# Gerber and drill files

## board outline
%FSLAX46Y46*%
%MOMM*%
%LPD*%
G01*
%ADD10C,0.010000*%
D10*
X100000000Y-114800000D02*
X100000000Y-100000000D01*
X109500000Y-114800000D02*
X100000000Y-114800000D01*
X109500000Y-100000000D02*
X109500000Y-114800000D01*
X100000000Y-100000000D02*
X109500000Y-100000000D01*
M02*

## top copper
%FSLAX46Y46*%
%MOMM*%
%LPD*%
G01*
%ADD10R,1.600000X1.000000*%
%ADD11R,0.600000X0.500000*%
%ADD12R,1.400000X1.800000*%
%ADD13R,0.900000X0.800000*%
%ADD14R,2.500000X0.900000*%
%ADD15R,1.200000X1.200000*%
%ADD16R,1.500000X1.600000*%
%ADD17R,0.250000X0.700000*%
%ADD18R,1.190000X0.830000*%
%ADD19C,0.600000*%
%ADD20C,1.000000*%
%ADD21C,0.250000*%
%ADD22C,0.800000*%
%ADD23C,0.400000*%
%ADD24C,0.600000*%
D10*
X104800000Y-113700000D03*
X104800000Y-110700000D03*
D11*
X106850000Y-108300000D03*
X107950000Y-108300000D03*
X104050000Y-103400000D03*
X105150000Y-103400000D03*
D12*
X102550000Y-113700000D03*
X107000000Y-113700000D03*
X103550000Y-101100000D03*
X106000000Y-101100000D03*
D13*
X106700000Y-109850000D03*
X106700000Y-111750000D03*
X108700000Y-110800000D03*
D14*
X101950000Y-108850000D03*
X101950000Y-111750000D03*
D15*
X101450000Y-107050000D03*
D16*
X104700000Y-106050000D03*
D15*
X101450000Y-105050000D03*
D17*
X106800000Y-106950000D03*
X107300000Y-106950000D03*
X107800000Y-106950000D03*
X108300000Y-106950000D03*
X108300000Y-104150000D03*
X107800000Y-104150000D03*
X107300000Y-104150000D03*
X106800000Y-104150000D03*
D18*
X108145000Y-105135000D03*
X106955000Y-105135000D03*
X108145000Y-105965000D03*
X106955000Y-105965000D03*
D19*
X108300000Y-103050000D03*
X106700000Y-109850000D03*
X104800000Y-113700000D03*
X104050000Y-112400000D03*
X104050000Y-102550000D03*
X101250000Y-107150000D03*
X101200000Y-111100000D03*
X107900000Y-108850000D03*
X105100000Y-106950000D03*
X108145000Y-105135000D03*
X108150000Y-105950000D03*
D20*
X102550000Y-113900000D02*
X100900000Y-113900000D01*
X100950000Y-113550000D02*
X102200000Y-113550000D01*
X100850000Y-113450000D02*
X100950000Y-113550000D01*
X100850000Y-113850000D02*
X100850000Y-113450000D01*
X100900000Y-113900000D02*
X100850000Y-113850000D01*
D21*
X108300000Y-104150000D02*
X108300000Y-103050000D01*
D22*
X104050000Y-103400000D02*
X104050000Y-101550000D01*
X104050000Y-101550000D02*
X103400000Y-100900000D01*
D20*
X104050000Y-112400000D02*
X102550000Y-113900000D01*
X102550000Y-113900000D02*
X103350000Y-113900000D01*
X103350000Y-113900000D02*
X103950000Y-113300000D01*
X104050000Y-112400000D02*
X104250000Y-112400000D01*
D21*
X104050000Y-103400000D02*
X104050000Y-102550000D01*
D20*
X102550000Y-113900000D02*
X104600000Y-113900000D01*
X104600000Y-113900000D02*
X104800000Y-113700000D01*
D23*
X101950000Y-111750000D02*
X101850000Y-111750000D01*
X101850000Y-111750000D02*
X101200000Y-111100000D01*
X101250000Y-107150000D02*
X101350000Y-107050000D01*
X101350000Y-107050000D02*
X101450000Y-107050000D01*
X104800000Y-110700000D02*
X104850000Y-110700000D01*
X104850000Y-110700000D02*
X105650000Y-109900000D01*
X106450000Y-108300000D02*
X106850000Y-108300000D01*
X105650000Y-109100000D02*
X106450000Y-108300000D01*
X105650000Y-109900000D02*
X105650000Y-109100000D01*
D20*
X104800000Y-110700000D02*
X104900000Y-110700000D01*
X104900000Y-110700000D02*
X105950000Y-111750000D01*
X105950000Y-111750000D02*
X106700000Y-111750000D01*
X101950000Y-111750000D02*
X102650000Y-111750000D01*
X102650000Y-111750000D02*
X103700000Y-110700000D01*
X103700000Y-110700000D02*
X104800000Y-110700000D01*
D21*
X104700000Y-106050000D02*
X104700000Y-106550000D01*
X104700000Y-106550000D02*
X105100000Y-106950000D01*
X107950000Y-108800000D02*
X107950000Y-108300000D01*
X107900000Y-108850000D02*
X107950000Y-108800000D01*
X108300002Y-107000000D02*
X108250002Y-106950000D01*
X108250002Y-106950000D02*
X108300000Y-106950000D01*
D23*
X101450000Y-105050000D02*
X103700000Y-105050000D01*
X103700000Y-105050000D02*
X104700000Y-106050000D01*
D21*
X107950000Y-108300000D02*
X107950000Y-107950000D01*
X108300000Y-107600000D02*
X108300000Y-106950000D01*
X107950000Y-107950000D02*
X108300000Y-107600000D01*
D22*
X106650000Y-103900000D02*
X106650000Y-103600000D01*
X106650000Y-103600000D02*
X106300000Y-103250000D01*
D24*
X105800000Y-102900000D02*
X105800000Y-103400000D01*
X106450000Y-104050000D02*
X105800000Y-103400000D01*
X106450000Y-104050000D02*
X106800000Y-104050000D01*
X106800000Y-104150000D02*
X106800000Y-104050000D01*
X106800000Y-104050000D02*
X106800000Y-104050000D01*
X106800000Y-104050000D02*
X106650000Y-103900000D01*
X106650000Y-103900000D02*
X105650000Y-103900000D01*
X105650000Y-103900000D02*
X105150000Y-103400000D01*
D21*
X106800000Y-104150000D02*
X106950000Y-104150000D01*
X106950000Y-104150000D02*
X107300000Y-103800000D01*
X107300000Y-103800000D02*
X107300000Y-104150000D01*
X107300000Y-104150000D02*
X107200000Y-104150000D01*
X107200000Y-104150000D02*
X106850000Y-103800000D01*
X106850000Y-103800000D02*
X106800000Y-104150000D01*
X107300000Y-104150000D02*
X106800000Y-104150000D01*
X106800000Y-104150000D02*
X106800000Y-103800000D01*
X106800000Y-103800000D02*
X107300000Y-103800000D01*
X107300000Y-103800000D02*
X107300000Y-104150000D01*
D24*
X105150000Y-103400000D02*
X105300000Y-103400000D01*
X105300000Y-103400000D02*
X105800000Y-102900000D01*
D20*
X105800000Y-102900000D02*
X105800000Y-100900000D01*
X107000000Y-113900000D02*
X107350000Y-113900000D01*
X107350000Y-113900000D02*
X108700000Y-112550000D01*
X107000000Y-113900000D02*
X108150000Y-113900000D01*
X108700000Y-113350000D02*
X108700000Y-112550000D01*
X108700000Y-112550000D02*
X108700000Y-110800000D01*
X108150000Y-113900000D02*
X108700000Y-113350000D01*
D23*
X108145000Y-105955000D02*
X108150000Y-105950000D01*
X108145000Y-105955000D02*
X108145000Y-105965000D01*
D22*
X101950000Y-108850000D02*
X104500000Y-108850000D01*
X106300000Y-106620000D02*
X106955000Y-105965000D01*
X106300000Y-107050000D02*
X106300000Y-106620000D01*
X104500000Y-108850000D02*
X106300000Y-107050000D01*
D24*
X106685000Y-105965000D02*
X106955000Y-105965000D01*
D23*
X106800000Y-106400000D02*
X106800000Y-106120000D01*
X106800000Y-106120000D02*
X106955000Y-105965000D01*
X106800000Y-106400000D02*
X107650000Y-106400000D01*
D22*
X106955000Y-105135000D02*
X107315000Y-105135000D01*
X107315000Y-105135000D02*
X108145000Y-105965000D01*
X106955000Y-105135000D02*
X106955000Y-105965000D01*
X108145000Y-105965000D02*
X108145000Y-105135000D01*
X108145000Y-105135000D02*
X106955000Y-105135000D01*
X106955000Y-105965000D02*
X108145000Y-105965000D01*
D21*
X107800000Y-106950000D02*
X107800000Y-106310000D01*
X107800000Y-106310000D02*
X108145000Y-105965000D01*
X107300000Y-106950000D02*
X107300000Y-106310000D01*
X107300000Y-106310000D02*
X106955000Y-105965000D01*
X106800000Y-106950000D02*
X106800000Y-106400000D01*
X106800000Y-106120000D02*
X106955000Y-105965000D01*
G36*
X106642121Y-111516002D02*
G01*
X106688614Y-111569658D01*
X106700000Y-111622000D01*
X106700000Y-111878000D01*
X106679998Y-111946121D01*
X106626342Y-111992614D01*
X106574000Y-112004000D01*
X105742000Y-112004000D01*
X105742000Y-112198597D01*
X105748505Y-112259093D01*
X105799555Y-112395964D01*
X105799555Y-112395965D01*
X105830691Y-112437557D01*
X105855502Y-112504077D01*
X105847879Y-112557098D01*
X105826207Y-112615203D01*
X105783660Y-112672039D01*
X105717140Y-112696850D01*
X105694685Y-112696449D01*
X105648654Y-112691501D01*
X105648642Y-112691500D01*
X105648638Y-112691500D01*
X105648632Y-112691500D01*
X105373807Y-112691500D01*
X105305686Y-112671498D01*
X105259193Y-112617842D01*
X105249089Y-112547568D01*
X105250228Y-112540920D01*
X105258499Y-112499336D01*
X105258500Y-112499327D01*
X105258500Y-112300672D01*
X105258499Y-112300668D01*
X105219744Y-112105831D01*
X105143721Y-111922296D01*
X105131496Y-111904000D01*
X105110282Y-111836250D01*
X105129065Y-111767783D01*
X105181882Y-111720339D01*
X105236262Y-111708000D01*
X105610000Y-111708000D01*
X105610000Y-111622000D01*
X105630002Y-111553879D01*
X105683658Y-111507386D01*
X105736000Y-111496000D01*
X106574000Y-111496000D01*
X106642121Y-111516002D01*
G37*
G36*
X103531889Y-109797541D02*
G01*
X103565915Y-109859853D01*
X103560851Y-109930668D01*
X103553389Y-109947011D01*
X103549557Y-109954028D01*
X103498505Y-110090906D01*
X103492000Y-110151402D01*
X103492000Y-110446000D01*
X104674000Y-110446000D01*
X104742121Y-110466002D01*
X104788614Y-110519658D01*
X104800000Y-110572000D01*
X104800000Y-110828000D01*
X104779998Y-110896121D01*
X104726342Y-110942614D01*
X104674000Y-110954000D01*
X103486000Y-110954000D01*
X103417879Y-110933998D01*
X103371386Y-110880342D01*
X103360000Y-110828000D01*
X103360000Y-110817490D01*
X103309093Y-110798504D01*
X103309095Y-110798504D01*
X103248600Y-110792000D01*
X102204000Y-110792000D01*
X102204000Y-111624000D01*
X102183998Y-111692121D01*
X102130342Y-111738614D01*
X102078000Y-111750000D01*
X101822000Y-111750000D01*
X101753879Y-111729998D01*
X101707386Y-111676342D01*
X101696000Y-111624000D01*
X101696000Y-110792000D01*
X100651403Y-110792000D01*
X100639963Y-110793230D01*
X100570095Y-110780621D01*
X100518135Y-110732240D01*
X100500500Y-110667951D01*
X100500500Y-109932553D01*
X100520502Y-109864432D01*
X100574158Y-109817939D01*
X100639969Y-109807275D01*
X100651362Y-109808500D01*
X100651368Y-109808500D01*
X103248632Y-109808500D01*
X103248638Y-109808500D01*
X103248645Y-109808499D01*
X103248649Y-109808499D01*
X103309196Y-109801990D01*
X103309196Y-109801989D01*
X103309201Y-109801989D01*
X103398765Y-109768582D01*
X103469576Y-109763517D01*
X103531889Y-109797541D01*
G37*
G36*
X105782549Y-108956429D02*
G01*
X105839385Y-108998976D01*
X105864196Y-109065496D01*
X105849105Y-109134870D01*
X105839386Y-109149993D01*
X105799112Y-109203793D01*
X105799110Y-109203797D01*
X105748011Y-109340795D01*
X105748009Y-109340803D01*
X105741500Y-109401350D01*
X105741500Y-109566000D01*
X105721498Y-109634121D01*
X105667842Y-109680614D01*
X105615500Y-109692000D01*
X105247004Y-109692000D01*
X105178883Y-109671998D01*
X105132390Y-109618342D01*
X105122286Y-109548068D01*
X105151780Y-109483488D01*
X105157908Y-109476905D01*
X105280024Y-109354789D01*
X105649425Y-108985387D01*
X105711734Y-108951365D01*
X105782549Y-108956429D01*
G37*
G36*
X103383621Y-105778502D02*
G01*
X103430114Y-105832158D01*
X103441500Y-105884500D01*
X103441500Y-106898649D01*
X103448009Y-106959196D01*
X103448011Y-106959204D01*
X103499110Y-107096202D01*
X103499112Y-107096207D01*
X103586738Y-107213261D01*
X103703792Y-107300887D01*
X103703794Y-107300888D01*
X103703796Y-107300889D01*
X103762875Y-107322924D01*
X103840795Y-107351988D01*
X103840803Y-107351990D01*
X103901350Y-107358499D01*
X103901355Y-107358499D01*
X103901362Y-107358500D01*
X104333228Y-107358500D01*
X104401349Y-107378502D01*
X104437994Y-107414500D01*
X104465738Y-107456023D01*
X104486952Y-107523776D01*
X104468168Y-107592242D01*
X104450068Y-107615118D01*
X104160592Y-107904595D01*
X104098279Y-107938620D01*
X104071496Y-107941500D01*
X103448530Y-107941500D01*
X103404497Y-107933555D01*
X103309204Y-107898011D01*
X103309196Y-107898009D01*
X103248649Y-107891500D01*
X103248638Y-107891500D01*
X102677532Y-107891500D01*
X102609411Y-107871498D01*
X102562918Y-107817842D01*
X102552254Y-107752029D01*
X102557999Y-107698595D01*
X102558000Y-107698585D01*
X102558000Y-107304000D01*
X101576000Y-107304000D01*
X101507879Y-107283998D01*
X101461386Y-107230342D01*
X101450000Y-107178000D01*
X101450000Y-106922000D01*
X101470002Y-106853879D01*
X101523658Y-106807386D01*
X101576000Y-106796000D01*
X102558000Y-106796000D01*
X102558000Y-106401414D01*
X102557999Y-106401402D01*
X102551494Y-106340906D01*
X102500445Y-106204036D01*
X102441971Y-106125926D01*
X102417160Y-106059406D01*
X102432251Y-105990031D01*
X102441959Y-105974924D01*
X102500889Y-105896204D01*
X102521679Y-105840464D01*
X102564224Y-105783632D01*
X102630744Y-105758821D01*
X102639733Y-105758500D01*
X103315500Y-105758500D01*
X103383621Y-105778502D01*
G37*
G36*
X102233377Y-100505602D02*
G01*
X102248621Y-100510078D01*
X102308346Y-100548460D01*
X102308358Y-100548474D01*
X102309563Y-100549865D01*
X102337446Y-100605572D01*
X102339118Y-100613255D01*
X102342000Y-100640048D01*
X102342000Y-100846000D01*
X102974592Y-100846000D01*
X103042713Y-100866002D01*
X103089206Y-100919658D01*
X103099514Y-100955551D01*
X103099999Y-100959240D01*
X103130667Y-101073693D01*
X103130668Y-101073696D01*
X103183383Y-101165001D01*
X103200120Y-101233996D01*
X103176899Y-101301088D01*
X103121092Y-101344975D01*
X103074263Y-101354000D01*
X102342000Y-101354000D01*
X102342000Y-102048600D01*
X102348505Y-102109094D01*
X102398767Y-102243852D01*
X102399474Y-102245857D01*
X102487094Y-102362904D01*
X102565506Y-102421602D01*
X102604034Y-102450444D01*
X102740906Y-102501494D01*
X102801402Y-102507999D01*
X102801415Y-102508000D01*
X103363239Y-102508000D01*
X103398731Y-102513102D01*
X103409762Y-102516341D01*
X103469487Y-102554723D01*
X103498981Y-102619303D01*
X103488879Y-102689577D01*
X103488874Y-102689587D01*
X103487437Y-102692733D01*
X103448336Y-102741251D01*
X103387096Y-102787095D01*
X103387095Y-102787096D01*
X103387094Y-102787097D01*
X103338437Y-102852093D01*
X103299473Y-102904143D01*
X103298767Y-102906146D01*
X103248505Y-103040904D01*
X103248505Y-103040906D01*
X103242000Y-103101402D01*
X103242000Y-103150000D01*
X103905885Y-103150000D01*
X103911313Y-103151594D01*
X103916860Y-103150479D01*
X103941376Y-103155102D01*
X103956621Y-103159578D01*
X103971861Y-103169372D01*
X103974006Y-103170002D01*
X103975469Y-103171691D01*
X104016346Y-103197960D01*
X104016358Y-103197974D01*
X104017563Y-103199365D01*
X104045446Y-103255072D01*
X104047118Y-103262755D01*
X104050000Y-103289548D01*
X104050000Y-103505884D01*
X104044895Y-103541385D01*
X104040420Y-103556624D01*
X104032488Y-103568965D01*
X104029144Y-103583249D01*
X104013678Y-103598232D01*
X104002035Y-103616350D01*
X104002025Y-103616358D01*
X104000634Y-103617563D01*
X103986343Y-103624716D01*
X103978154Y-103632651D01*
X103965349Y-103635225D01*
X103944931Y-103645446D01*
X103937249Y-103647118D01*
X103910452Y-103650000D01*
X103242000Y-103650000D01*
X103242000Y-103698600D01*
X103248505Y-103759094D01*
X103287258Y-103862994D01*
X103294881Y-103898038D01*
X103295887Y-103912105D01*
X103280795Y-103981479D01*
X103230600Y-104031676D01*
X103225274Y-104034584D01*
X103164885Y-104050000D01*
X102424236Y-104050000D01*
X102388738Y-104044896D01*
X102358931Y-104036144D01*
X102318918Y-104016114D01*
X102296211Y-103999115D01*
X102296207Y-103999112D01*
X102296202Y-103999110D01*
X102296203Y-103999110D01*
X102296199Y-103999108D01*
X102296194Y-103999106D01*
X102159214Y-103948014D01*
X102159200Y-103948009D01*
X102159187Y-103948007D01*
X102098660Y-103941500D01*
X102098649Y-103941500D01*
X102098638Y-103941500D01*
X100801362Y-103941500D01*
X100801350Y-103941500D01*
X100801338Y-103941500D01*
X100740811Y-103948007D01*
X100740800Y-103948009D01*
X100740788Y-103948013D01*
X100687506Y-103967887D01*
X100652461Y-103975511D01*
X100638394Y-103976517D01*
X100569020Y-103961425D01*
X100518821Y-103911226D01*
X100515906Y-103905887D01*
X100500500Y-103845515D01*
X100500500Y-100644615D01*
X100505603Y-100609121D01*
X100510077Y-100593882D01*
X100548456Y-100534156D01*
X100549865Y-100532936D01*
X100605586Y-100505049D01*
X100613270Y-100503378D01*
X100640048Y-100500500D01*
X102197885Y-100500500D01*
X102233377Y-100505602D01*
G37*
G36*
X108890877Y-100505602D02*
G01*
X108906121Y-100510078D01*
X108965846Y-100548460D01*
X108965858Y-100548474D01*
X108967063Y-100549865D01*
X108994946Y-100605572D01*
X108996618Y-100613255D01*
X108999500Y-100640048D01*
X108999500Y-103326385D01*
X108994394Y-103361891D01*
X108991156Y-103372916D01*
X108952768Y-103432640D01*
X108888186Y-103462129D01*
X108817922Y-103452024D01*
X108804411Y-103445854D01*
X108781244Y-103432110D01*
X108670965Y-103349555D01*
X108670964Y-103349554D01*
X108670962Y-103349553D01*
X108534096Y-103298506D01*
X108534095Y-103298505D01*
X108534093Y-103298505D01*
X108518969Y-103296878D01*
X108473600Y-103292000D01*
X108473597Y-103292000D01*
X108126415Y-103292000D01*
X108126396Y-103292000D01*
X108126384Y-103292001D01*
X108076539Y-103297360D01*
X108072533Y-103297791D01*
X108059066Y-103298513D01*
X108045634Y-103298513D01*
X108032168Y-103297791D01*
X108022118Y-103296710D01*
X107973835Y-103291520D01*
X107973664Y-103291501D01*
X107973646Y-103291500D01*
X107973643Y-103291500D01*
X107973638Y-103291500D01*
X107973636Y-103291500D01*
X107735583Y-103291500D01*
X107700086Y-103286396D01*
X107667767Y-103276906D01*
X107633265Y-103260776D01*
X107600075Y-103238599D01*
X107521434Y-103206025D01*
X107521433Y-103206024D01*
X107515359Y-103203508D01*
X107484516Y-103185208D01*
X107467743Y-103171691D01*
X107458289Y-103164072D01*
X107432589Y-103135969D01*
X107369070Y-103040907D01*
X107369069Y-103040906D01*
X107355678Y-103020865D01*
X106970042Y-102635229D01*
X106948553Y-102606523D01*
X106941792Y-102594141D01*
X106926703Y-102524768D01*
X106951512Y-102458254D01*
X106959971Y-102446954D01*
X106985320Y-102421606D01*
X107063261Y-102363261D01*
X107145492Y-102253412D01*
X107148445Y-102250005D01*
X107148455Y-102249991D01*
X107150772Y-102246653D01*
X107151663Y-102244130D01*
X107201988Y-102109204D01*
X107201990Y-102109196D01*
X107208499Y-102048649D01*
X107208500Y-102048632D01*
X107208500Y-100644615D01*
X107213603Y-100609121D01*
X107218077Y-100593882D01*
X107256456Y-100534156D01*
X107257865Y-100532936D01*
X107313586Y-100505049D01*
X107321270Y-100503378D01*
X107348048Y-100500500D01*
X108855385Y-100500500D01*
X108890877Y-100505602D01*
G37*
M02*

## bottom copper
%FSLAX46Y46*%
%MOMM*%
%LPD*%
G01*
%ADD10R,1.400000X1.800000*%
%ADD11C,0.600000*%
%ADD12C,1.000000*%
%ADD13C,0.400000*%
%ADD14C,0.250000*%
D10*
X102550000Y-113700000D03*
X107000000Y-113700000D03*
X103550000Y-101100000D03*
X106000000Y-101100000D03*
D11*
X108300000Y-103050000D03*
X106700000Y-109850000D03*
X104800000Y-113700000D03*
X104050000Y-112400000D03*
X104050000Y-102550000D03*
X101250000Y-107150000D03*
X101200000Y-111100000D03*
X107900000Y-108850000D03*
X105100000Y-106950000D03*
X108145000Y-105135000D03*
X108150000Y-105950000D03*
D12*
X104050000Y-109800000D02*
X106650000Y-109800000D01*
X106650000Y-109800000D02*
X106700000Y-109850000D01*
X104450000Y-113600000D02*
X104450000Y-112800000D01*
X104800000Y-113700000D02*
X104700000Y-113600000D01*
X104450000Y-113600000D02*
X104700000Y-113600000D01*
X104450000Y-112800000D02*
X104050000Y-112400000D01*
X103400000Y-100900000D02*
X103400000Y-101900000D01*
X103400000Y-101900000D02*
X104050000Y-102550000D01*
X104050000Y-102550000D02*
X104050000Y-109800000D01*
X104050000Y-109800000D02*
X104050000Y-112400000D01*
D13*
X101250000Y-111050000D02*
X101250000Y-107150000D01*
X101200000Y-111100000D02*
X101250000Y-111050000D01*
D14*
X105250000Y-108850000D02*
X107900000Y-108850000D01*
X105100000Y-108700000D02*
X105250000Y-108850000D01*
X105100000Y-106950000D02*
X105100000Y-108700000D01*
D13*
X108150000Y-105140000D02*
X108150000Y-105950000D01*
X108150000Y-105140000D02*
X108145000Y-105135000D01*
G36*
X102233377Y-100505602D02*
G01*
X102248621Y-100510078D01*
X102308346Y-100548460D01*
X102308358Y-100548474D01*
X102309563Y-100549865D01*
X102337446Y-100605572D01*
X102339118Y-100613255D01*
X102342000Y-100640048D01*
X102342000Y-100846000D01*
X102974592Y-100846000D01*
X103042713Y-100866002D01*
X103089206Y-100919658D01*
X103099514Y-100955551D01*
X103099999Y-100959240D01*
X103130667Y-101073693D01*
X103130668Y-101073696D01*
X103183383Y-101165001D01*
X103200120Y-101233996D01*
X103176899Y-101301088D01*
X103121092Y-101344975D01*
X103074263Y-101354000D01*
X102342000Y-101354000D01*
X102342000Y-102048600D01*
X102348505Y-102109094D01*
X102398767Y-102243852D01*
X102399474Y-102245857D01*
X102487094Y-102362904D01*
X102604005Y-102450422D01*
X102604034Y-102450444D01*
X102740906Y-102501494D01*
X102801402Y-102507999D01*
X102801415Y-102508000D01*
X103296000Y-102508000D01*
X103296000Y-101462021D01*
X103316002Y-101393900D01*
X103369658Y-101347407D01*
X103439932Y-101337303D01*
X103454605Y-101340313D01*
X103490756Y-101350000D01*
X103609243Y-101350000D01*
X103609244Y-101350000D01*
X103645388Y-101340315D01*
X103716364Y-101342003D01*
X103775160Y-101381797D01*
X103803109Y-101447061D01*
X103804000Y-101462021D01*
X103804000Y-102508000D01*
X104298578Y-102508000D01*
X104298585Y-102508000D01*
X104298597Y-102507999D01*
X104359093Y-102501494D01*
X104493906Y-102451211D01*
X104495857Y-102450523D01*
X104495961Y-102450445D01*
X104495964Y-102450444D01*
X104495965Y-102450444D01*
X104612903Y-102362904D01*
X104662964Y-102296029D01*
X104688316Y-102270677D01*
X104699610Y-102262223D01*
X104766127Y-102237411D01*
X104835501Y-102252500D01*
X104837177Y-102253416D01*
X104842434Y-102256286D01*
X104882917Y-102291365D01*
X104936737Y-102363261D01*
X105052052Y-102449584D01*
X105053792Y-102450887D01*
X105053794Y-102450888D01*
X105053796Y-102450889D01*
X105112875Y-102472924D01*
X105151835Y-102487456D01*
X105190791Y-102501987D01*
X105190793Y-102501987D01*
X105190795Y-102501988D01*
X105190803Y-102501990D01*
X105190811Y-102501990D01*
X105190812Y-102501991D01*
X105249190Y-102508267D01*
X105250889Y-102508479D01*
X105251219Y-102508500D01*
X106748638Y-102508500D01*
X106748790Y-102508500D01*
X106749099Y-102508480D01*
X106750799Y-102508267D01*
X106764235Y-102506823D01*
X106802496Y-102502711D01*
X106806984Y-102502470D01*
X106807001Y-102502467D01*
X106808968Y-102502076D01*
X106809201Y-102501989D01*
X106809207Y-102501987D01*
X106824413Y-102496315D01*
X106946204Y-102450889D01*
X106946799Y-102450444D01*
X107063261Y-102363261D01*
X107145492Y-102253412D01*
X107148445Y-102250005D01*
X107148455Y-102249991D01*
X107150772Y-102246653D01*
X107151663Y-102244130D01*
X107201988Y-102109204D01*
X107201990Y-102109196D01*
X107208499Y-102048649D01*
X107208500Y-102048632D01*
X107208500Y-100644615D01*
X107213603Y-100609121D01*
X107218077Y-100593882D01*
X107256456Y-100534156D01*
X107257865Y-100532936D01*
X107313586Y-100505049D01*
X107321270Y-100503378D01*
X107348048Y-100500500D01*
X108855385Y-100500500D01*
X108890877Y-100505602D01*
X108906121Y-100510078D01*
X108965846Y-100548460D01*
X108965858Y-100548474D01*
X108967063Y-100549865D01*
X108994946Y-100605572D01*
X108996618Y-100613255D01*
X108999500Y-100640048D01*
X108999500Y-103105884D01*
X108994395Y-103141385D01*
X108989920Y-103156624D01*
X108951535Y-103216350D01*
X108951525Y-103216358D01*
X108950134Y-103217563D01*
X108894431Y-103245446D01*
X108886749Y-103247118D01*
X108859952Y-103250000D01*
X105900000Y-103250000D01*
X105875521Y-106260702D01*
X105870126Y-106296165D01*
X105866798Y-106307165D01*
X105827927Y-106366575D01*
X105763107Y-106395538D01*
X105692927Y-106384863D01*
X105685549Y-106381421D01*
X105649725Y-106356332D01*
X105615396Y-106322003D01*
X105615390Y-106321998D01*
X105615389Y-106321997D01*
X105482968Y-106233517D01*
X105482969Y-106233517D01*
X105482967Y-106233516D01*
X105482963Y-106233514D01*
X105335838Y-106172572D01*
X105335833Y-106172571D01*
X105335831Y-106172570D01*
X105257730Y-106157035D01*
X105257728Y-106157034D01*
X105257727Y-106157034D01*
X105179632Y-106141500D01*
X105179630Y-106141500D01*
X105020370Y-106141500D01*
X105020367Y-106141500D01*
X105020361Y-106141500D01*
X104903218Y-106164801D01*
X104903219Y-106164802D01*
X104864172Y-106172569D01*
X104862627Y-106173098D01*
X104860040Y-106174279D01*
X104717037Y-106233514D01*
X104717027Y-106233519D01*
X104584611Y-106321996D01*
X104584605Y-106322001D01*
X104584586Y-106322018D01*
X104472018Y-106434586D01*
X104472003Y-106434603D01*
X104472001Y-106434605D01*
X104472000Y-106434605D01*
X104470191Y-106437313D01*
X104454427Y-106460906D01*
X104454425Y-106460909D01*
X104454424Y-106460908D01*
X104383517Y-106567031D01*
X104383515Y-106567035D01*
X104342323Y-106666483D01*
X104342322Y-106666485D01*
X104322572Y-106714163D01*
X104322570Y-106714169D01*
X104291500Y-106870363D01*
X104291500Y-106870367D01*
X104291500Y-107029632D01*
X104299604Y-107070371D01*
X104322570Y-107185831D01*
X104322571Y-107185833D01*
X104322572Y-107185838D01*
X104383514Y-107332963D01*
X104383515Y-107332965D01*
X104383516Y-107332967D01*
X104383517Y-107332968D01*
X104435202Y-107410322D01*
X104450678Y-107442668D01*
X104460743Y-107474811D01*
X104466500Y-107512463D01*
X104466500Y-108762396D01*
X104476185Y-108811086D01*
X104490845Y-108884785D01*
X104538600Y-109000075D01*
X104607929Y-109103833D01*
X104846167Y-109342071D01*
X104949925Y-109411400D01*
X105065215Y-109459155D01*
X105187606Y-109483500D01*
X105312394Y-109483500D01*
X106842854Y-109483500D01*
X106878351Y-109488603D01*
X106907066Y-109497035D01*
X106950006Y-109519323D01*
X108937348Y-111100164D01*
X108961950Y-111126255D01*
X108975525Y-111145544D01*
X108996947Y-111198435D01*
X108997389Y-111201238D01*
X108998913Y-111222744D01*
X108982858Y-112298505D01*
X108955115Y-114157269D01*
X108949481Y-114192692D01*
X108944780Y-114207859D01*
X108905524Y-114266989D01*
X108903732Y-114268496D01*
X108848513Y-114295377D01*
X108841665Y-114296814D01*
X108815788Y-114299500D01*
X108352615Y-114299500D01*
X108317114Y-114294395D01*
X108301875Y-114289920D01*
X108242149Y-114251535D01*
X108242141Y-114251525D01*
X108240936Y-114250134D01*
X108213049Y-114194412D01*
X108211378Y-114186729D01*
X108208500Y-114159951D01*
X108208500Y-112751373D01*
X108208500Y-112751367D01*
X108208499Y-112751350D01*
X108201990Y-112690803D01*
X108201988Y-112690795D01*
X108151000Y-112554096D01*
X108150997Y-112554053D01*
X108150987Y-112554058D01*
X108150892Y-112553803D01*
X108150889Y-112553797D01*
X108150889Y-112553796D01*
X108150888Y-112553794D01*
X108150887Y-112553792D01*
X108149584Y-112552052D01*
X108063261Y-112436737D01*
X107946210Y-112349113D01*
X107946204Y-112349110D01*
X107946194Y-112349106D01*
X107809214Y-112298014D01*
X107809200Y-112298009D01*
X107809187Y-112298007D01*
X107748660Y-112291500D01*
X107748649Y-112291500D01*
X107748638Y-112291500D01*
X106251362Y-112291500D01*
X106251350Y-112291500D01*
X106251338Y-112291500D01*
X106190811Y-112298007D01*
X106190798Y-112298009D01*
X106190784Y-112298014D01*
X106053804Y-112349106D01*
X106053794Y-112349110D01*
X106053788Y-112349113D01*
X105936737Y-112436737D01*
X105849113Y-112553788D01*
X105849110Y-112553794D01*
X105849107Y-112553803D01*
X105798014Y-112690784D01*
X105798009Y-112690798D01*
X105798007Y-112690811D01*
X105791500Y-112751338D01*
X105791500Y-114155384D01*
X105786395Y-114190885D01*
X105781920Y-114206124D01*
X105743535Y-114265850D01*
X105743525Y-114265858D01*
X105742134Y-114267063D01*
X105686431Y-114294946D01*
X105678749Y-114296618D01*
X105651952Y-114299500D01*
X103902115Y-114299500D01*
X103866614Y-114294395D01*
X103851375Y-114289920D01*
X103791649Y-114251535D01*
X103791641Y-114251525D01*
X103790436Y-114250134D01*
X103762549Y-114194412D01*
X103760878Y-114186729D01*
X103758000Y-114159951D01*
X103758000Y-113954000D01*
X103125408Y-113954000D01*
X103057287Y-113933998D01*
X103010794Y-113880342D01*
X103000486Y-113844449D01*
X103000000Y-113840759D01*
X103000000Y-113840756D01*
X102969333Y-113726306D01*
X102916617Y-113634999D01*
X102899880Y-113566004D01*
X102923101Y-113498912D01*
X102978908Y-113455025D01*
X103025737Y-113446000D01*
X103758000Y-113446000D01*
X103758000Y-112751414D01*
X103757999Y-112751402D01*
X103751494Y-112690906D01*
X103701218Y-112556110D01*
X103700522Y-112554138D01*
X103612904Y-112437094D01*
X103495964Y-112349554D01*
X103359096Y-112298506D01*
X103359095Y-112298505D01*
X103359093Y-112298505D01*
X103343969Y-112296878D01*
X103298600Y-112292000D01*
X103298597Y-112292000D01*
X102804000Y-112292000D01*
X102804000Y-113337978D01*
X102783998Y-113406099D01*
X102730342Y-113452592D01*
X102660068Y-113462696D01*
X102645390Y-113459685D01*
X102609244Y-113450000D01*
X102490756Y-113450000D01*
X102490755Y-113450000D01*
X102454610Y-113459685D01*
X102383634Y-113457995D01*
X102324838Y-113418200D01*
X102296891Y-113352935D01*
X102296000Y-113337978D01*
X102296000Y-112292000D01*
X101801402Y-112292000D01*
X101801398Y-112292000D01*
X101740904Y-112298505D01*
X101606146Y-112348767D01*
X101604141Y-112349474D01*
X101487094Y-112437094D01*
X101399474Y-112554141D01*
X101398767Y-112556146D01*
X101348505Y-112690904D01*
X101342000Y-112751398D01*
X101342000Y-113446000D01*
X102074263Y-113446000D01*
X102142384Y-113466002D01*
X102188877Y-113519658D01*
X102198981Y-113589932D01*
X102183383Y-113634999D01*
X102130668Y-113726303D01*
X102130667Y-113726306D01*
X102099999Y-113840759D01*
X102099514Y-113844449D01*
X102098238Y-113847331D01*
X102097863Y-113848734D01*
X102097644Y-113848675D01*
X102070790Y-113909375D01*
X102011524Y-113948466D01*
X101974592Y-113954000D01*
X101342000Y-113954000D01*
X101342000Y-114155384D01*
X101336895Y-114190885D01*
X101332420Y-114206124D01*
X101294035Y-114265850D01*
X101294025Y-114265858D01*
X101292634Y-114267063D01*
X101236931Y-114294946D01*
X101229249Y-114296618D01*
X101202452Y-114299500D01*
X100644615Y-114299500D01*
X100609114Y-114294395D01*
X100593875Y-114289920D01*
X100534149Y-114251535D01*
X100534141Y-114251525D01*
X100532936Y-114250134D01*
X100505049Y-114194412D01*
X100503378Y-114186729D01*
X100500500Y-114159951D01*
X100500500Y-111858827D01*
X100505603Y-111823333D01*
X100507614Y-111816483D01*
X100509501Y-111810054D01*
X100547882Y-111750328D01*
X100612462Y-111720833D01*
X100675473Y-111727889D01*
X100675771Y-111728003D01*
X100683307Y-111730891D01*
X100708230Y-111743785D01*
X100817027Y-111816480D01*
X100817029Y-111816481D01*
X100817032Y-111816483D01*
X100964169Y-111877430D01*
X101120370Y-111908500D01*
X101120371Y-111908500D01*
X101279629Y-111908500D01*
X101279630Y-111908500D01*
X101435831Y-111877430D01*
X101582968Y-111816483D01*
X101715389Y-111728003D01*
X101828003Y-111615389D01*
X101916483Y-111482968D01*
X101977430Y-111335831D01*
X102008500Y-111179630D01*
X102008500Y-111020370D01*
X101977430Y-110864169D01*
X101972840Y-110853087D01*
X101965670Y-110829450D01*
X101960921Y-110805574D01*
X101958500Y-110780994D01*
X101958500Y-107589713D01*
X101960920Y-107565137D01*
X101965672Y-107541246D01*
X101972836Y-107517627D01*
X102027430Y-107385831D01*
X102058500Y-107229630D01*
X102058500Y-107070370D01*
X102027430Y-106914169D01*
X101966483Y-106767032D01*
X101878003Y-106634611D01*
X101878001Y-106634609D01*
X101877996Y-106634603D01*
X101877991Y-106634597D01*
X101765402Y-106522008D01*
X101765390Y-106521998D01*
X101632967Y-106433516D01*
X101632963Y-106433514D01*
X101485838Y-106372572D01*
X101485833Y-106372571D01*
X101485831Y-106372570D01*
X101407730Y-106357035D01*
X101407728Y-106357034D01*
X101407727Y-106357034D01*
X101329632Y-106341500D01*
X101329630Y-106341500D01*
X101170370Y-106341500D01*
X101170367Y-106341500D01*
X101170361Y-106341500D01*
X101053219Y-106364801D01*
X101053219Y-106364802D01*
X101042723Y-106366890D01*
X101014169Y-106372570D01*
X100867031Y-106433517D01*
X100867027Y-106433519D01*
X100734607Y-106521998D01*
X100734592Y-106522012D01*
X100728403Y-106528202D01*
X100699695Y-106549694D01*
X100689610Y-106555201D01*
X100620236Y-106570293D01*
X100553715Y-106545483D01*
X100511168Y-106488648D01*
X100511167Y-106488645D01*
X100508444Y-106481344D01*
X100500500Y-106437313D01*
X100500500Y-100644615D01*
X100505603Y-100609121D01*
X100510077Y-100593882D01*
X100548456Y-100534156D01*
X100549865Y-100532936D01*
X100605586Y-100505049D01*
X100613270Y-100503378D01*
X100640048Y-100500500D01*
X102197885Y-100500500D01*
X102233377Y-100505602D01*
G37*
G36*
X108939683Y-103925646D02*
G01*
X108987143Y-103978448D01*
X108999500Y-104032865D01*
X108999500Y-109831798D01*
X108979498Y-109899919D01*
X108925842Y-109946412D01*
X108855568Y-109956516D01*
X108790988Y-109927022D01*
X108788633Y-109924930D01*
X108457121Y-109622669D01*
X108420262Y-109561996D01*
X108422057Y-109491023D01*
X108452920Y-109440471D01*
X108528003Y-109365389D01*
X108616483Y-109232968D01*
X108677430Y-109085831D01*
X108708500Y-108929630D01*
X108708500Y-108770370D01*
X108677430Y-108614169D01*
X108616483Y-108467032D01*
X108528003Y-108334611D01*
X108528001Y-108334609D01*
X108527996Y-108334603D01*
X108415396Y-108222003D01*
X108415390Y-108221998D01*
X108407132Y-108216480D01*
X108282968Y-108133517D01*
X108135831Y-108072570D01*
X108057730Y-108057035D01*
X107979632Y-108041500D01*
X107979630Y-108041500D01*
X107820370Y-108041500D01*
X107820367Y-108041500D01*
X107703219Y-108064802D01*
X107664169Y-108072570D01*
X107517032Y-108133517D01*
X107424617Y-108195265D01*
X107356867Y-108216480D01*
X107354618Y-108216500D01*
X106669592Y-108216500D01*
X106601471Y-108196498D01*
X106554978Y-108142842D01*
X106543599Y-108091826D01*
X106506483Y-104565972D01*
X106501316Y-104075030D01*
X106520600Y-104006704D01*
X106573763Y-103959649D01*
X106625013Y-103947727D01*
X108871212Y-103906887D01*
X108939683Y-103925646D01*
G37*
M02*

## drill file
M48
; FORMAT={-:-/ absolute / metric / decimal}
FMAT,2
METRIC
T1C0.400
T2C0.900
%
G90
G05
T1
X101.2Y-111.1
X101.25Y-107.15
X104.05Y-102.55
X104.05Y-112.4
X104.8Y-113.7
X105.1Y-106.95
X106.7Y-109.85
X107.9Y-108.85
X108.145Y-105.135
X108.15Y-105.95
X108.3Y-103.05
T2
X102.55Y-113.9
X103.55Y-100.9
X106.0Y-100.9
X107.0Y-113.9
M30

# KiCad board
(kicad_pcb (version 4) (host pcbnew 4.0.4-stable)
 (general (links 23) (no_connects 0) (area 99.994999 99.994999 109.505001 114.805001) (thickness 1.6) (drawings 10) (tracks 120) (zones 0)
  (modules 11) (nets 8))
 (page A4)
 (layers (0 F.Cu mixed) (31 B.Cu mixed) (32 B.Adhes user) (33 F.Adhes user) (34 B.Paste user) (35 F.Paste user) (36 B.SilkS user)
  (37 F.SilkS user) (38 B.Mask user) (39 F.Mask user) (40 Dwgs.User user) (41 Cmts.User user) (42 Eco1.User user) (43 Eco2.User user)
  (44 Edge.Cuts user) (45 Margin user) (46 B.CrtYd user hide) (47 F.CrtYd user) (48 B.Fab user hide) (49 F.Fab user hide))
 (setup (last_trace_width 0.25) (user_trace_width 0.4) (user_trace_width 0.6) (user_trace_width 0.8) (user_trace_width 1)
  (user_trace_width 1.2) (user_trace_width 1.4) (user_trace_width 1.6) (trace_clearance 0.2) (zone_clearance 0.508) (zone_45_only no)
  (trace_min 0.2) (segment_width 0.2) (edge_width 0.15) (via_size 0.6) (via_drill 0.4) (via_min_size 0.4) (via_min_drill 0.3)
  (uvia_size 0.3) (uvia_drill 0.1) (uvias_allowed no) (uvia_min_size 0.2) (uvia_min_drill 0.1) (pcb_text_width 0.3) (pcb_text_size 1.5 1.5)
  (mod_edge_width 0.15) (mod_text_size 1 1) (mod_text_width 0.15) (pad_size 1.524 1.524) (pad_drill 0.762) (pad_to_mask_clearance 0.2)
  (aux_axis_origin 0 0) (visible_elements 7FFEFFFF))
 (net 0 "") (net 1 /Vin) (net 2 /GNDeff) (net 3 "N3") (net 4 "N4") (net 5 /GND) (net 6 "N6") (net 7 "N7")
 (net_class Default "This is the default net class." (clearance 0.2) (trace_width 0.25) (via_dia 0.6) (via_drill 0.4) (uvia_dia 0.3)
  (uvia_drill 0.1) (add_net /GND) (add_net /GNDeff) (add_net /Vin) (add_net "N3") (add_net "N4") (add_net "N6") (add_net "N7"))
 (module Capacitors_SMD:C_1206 (layer F.Cu) (at 104.8 112.2 90)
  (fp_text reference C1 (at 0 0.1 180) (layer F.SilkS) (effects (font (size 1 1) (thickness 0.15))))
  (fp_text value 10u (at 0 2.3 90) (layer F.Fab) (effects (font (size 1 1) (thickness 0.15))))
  (pad 1 smd rect (at -1.5 0 90) (size 1 1.6) (layers F.Cu F.Paste F.Mask) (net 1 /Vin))
  (pad 2 smd rect (at 1.5 0 90) (size 1 1.6) (layers F.Cu F.Paste F.Mask) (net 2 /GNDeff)))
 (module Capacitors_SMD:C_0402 (layer F.Cu) (at 107.4 108.3)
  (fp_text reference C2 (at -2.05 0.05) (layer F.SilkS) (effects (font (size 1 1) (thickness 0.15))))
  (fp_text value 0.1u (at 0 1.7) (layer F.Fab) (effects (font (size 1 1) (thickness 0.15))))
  (pad 1 smd rect (at -0.55 0) (size 0.6 0.5) (layers F.Cu F.Paste F.Mask) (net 2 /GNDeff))
  (pad 2 smd rect (at 0.55 0) (size 0.6 0.5) (layers F.Cu F.Paste F.Mask) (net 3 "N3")))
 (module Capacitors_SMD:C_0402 (layer F.Cu) (at 104.6 103.4)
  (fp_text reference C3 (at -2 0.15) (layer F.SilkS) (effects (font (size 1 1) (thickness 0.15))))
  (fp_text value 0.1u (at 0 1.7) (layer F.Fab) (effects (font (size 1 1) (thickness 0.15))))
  (pad 1 smd rect (at -0.55 0) (size 0.6 0.5) (layers F.Cu F.Paste F.Mask) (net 1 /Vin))
  (pad 2 smd rect (at 0.55 0) (size 0.6 0.5) (layers F.Cu F.Paste F.Mask) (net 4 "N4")))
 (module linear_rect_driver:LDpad (layer F.Cu) (at 103 113.85 270)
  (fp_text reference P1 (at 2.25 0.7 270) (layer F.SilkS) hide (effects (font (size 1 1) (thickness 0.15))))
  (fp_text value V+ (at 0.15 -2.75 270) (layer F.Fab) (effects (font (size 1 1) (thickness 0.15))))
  (pad 1 thru_hole rect (at 0.05 0.45 270) (size 1.8 1.4) (drill 0.9 (offset -0.2 0)) (layers *.Cu *.Mask) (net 1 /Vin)))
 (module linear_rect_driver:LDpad (layer F.Cu) (at 107.45 113.85 270)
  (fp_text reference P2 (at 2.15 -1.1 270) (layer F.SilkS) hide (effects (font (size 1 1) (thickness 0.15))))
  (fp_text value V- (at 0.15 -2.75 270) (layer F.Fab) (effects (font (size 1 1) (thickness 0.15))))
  (pad 1 thru_hole rect (at 0.05 0.45 270) (size 1.8 1.4) (drill 0.9 (offset -0.2 0)) (layers *.Cu *.Mask) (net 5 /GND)))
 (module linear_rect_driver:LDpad (layer F.Cu) (at 103.1 100.95 90)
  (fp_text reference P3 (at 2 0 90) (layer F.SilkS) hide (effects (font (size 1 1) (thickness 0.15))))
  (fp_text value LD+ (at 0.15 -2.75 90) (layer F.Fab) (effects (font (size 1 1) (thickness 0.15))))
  (pad 1 thru_hole rect (at 0.05 0.45 90) (size 1.8 1.4) (drill 0.9 (offset -0.2 0)) (layers *.Cu *.Mask) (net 1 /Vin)))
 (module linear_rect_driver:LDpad (layer F.Cu) (at 105.55 100.95 90)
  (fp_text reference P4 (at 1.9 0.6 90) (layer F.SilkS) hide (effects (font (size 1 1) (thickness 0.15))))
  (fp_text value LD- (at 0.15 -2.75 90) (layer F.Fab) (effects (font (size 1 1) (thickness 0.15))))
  (pad 1 thru_hole rect (at 0.05 0.45 90) (size 1.8 1.4) (drill 0.9 (offset -0.2 0)) (layers *.Cu *.Mask) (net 4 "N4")))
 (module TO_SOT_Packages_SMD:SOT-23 (layer F.Cu) (at 107.7 110.8)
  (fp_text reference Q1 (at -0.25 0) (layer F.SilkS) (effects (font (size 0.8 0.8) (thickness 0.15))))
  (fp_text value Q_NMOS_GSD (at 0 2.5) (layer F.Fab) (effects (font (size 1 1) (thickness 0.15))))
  (pad 1 smd rect (at -1 -0.95) (size 0.9 0.8) (layers F.Cu F.Paste F.Mask) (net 1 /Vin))
  (pad 2 smd rect (at -1 0.95) (size 0.9 0.8) (layers F.Cu F.Paste F.Mask) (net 2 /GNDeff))
  (pad 3 smd rect (at 1 0) (size 0.9 0.8) (layers F.Cu F.Paste F.Mask) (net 5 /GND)))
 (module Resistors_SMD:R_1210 (layer F.Cu) (at 101.95 110.3 270)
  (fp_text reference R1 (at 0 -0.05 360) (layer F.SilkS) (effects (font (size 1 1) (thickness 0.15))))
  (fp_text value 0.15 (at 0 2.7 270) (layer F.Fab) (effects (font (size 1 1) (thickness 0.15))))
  (pad 1 smd rect (at -1.45 0 270) (size 0.9 2.5) (layers F.Cu F.Paste F.Mask) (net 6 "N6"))
  (pad 2 smd rect (at 1.45 0 270) (size 0.9 2.5) (layers F.Cu F.Paste F.Mask) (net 2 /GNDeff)))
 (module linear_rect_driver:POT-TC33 (layer F.Cu) (at 103.95 106.05 270)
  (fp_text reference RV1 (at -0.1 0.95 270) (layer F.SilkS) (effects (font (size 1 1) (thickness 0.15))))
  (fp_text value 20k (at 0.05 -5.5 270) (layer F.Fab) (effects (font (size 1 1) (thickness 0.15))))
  (pad 3 smd rect (at 1 2.5 270) (size 1.2 1.2) (layers F.Cu F.Paste F.Mask) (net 2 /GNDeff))
  (pad 2 smd rect (at 0 -0.75 270) (size 1.6 1.5) (layers F.Cu F.Paste F.Mask) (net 3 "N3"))
  (pad 1 smd rect (at -1 2.5 270) (size 1.2 1.2) (layers F.Cu F.Paste F.Mask) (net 3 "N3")))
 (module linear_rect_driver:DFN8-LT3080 (layer F.Cu) (at 107.55 105.55 90)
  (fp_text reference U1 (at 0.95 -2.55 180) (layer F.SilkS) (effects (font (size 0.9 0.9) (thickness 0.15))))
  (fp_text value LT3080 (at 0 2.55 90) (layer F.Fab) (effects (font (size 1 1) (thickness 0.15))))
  (pad 1 smd rect (at -1.4 -0.75 90) (size 0.7 0.25) (layers F.Cu F.Paste F.Mask) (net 6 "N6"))
  (pad 1 smd rect (at -1.4 -0.25 90) (size 0.7 0.25) (layers F.Cu F.Paste F.Mask) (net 6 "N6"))
  (pad 1 smd rect (at -1.4 0.25 90) (size 0.7 0.25) (layers F.Cu F.Paste F.Mask) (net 6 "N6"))
  (pad 2 smd rect (at -1.4 0.75 90) (size 0.7 0.25) (layers F.Cu F.Paste F.Mask) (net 3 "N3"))
  (pad 3 smd rect (at 1.4 0.75 90) (size 0.7 0.25) (layers F.Cu F.Paste F.Mask) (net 1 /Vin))
  (pad 5 smd rect (at 1.4 0.25 90) (size 0.7 0.25) (layers F.Cu F.Paste F.Mask) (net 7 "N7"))
  (pad 4 smd rect (at 1.4 -0.25 90) (size 0.7 0.25) (layers F.Cu F.Paste F.Mask) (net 4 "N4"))
  (pad 4 smd rect (at 1.4 -0.75 90) (size 0.7 0.25) (layers F.Cu F.Paste F.Mask) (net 4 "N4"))
  (pad 1 smd rect (at 0.415 0.595 90) (size 0.83 1.19) (layers F.Cu F.Paste F.Mask) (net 6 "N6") (solder_paste_margin_ratio -0.2))
  (pad 1 smd rect (at 0.415 -0.595 90) (size 0.83 1.19) (layers F.Cu F.Paste F.Mask) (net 6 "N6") (solder_paste_margin_ratio -0.2))
  (pad 1 smd rect (at -0.415 0.595 90) (size 0.83 1.19) (layers F.Cu F.Paste F.Mask) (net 6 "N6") (solder_paste_margin_ratio -0.2))
  (pad 1 smd rect (at -0.415 -0.595 90) (size 0.83 1.19) (layers F.Cu F.Paste F.Mask) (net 6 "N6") (solder_paste_margin_ratio -0.2)))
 (gr_line (start 100 114.8) (end 100 100) (angle 90) (layer Edge.Cuts) (width 0.01))
 (gr_line (start 109.5 114.8) (end 100 114.8) (angle 90) (layer Edge.Cuts) (width 0.01))
 (gr_line (start 109.5 100) (end 109.5 114.8) (angle 90) (layer Edge.Cuts) (width 0.01))
 (gr_line (start 100 100) (end 109.5 100) (angle 90) (layer Edge.Cuts) (width 0.01))
 (segment (start 102.55 113.9) (end 100.9 113.9) (width 1) (layer F.Cu) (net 1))
 (segment (start 100.95 113.55) (end 102.2 113.55) (width 1) (layer F.Cu) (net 1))
 (segment (start 100.85 113.45) (end 100.95 113.55) (width 1) (layer F.Cu) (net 1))
 (segment (start 100.85 113.85) (end 100.85 113.45) (width 1) (layer F.Cu) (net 1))
 (segment (start 100.9 113.9) (end 100.85 113.85) (width 1) (layer F.Cu) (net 1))
 (segment (start 108.3 104.15) (end 108.3 103.05) (width 0.25) (layer F.Cu) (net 1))
 (via (at 108.3 103.05) (size 0.6) (drill 0.4) (layers F.Cu B.Cu) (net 1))
 (segment (start 104.05 103.4) (end 104.05 101.55) (width 0.8) (layer F.Cu) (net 1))
 (segment (start 104.05 101.55) (end 103.4 100.9) (width 0.8) (layer F.Cu) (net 1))
 (via (at 106.7 109.85) (size 0.6) (drill 0.4) (layers F.Cu B.Cu) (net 1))
 (segment (start 104.05 109.8) (end 106.65 109.8) (width 1) (layer B.Cu) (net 1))
 (segment (start 106.65 109.8) (end 106.7 109.85) (width 1) (layer B.Cu) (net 1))
 (segment (start 104.45 113.6) (end 104.45 112.8) (width 1) (layer B.Cu) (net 1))
 (segment (start 104.8 113.7) (end 104.7 113.6) (width 1) (layer B.Cu) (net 1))
 (segment (start 104.45 113.6) (end 104.7 113.6) (width 1) (layer B.Cu) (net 1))
 (via (at 104.8 113.7) (size 0.6) (drill 0.4) (layers F.Cu B.Cu) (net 1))
 (segment (start 104.45 112.8) (end 104.05 112.4) (width 1) (layer B.Cu) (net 1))
 (segment (start 104.05 112.4) (end 102.55 113.9) (width 1) (layer F.Cu) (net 1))
 (segment (start 102.55 113.9) (end 103.35 113.9) (width 1) (layer F.Cu) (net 1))
 (segment (start 103.35 113.9) (end 103.95 113.3) (width 1) (layer F.Cu) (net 1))
 (via (at 104.05 112.4) (size 0.6) (drill 0.4) (layers F.Cu B.Cu) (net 1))
 (segment (start 104.05 112.4) (end 104.25 112.4) (width 1) (layer F.Cu) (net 1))
 (segment (start 103.4 100.9) (end 103.4 101.9) (width 1) (layer B.Cu) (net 1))
 (segment (start 103.4 101.9) (end 104.05 102.55) (width 1) (layer B.Cu) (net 1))
 (segment (start 104.05 102.55) (end 104.05 109.8) (width 1) (layer B.Cu) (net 1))
 (segment (start 104.05 109.8) (end 104.05 112.4) (width 1) (layer B.Cu) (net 1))
 (via (at 104.05 102.55) (size 0.6) (drill 0.4) (layers F.Cu B.Cu) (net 1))
 (segment (start 104.05 103.4) (end 104.05 102.55) (width 0.25) (layer F.Cu) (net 1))
 (segment (start 102.55 113.9) (end 104.6 113.9) (width 1) (layer F.Cu) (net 1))
 (segment (start 104.6 113.9) (end 104.8 113.7) (width 1) (layer F.Cu) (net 1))
 (segment (start 101.95 111.75) (end 101.85 111.75) (width 0.4) (layer F.Cu) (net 2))
 (segment (start 101.85 111.75) (end 101.2 111.1) (width 0.4) (layer F.Cu) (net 2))
 (segment (start 101.25 107.15) (end 101.35 107.05) (width 0.4) (layer F.Cu) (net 2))
 (via (at 101.25 107.15) (size 0.6) (drill 0.4) (layers F.Cu B.Cu) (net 2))
 (segment (start 101.25 111.05) (end 101.25 107.15) (width 0.4) (layer B.Cu) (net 2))
 (segment (start 101.2 111.1) (end 101.25 111.05) (width 0.4) (layer B.Cu) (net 2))
 (via (at 101.2 111.1) (size 0.6) (drill 0.4) (layers F.Cu B.Cu) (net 2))
 (segment (start 101.35 107.05) (end 101.45 107.05) (width 0.4) (layer F.Cu) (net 2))
 (segment (start 104.8 110.7) (end 104.85 110.7) (width 0.4) (layer F.Cu) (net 2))
 (segment (start 104.85 110.7) (end 105.65 109.9) (width 0.4) (layer F.Cu) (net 2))
 (segment (start 106.45 108.3) (end 106.85 108.3) (width 0.4) (layer F.Cu) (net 2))
 (segment (start 105.65 109.1) (end 106.45 108.3) (width 0.4) (layer F.Cu) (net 2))
 (segment (start 105.65 109.9) (end 105.65 109.1) (width 0.4) (layer F.Cu) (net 2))
 (segment (start 104.8 110.7) (end 104.9 110.7) (width 1) (layer F.Cu) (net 2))
 (segment (start 104.9 110.7) (end 105.95 111.75) (width 1) (layer F.Cu) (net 2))
 (segment (start 105.95 111.75) (end 106.7 111.75) (width 1) (layer F.Cu) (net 2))
 (segment (start 101.95 111.75) (end 102.65 111.75) (width 1) (layer F.Cu) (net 2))
 (segment (start 102.65 111.75) (end 103.7 110.7) (width 1) (layer F.Cu) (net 2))
 (segment (start 103.7 110.7) (end 104.8 110.7) (width 1) (layer F.Cu) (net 2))
 (segment (start 104.7 106.05) (end 104.7 106.55) (width 0.25) (layer F.Cu) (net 3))
 (segment (start 104.7 106.55) (end 105.1 106.95) (width 0.25) (layer F.Cu) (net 3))
 (segment (start 107.95 108.8) (end 107.95 108.3) (width 0.25) (layer F.Cu) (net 3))
 (segment (start 107.9 108.85) (end 107.95 108.8) (width 0.25) (layer F.Cu) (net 3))
 (via (at 107.9 108.85) (size 0.6) (drill 0.4) (layers F.Cu B.Cu) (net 3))
 (segment (start 105.25 108.85) (end 107.9 108.85) (width 0.25) (layer B.Cu) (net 3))
 (segment (start 105.1 108.7) (end 105.25 108.85) (width 0.25) (layer B.Cu) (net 3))
 (segment (start 105.1 106.95) (end 105.1 108.7) (width 0.25) (layer B.Cu) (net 3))
 (via (at 105.1 106.95) (size 0.6) (drill 0.4) (layers F.Cu B.Cu) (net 3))
 (segment (start 108.300002 107) (end 108.250002 106.95) (width 0.25) (layer F.Cu) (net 3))
 (segment (start 108.250002 106.95) (end 108.3 106.95) (width 0.25) (layer F.Cu) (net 3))
 (segment (start 101.45 105.05) (end 103.7 105.05) (width 0.4) (layer F.Cu) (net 3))
 (segment (start 103.7 105.05) (end 104.7 106.05) (width 0.4) (layer F.Cu) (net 3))
 (segment (start 107.95 108.3) (end 107.95 107.95) (width 0.25) (layer F.Cu) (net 3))
 (segment (start 108.3 107.6) (end 108.3 106.95) (width 0.25) (layer F.Cu) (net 3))
 (segment (start 107.95 107.95) (end 108.3 107.6) (width 0.25) (layer F.Cu) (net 3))
 (segment (start 106.65 103.9) (end 106.65 103.6) (width 0.8) (layer F.Cu) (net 4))
 (segment (start 106.65 103.6) (end 106.3 103.25) (width 0.8) (layer F.Cu) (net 4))
 (segment (start 105.8 102.9) (end 105.8 103.4) (width 0.6) (layer F.Cu) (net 4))
 (segment (start 106.45 104.05) (end 105.8 103.4) (width 0.6) (layer F.Cu) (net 4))
 (segment (start 106.45 104.05) (end 106.8 104.05) (width 0.6) (layer F.Cu) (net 4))
 (segment (start 106.8 104.15) (end 106.8 104.05) (width 0.6) (layer F.Cu) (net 4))
 (segment (start 106.8 104.05) (end 106.8 104.05) (width 0.6) (layer F.Cu) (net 4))
 (segment (start 106.8 104.05) (end 106.65 103.9) (width 0.6) (layer F.Cu) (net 4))
 (segment (start 106.65 103.9) (end 105.65 103.9) (width 0.6) (layer F.Cu) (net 4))
 (segment (start 105.65 103.9) (end 105.15 103.4) (width 0.6) (layer F.Cu) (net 4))
 (segment (start 106.8 104.15) (end 106.95 104.15) (width 0.25) (layer F.Cu) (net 4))
 (segment (start 106.95 104.15) (end 107.3 103.8) (width 0.25) (layer F.Cu) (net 4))
 (segment (start 107.3 103.8) (end 107.3 104.15) (width 0.25) (layer F.Cu) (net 4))
 (segment (start 107.3 104.15) (end 107.2 104.15) (width 0.25) (layer F.Cu) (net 4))
 (segment (start 107.2 104.15) (end 106.85 103.8) (width 0.25) (layer F.Cu) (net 4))
 (segment (start 106.85 103.8) (end 106.8 104.15) (width 0.25) (layer F.Cu) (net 4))
 (segment (start 107.3 104.15) (end 106.8 104.15) (width 0.25) (layer F.Cu) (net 4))
 (segment (start 106.8 104.15) (end 106.8 103.8) (width 0.25) (layer F.Cu) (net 4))
 (segment (start 106.8 103.8) (end 107.3 103.8) (width 0.25) (layer F.Cu) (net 4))
 (segment (start 107.3 103.8) (end 107.3 104.15) (width 0.25) (layer F.Cu) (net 4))
 (segment (start 105.15 103.4) (end 105.3 103.4) (width 0.6) (layer F.Cu) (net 4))
 (segment (start 105.3 103.4) (end 105.8 102.9) (width 0.6) (layer F.Cu) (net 4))
 (segment (start 105.8 102.9) (end 105.8 100.9) (width 1) (layer F.Cu) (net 4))
 (segment (start 107 113.9) (end 107.35 113.9) (width 1) (layer F.Cu) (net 5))
 (segment (start 107.35 113.9) (end 108.7 112.55) (width 1) (layer F.Cu) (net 5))
 (segment (start 107 113.9) (end 108.15 113.9) (width 1) (layer F.Cu) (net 5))
 (segment (start 108.7 113.35) (end 108.7 112.55) (width 1) (layer F.Cu) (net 5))
 (segment (start 108.7 112.55) (end 108.7 110.8) (width 1) (layer F.Cu) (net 5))
 (segment (start 108.15 113.9) (end 108.7 113.35) (width 1) (layer F.Cu) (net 5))
 (via (at 108.145 105.135) (size 0.6) (drill 0.4) (layers F.Cu B.Cu) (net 6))
 (segment (start 108.145 105.955) (end 108.15 105.95) (width 0.4) (layer F.Cu) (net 6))
 (via (at 108.15 105.95) (size 0.6) (drill 0.4) (layers F.Cu B.Cu) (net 6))
 (segment (start 108.15 105.14) (end 108.15 105.95) (width 0.4) (layer B.Cu) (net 6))
 (segment (start 108.15 105.14) (end 108.145 105.135) (width 0.4) (layer B.Cu) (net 6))
 (segment (start 108.145 105.955) (end 108.145 105.965) (width 0.4) (layer F.Cu) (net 6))
 (segment (start 101.95 108.85) (end 104.5 108.85) (width 0.8) (layer F.Cu) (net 6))
 (segment (start 106.3 106.62) (end 106.955 105.965) (width 0.8) (layer F.Cu) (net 6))
 (segment (start 106.3 107.05) (end 106.3 106.62) (width 0.8) (layer F.Cu) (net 6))
 (segment (start 104.5 108.85) (end 106.3 107.05) (width 0.8) (layer F.Cu) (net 6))
 (segment (start 106.685 105.965) (end 106.955 105.965) (width 0.6) (layer F.Cu) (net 6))
 (segment (start 106.8 106.4) (end 106.8 106.12) (width 0.4) (layer F.Cu) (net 6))
 (segment (start 106.8 106.12) (end 106.955 105.965) (width 0.4) (layer F.Cu) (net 6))
 (segment (start 106.8 106.4) (end 107.65 106.4) (width 0.4) (layer F.Cu) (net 6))
 (segment (start 106.955 105.135) (end 107.315 105.135) (width 0.8) (layer F.Cu) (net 6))
 (segment (start 107.315 105.135) (end 108.145 105.965) (width 0.8) (layer F.Cu) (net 6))
 (segment (start 106.955 105.135) (end 106.955 105.965) (width 0.8) (layer F.Cu) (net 6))
 (segment (start 108.145 105.965) (end 108.145 105.135) (width 0.8) (layer F.Cu) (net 6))
 (segment (start 108.145 105.135) (end 106.955 105.135) (width 0.8) (layer F.Cu) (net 6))
 (segment (start 106.955 105.965) (end 108.145 105.965) (width 0.8) (layer F.Cu) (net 6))
 (segment (start 107.8 106.95) (end 107.8 106.31) (width 0.25) (layer F.Cu) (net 6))
 (segment (start 107.8 106.31) (end 108.145 105.965) (width 0.25) (layer F.Cu) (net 6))
 (segment (start 107.3 106.95) (end 107.3 106.31) (width 0.25) (layer F.Cu) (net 6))
 (segment (start 107.3 106.31) (end 106.955 105.965) (width 0.25) (layer F.Cu) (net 6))
 (segment (start 106.8 106.95) (end 106.8 106.4) (width 0.25) (layer F.Cu) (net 6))
 (segment (start 106.8 106.12) (end 106.955 105.965) (width 0.25) (layer F.Cu) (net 6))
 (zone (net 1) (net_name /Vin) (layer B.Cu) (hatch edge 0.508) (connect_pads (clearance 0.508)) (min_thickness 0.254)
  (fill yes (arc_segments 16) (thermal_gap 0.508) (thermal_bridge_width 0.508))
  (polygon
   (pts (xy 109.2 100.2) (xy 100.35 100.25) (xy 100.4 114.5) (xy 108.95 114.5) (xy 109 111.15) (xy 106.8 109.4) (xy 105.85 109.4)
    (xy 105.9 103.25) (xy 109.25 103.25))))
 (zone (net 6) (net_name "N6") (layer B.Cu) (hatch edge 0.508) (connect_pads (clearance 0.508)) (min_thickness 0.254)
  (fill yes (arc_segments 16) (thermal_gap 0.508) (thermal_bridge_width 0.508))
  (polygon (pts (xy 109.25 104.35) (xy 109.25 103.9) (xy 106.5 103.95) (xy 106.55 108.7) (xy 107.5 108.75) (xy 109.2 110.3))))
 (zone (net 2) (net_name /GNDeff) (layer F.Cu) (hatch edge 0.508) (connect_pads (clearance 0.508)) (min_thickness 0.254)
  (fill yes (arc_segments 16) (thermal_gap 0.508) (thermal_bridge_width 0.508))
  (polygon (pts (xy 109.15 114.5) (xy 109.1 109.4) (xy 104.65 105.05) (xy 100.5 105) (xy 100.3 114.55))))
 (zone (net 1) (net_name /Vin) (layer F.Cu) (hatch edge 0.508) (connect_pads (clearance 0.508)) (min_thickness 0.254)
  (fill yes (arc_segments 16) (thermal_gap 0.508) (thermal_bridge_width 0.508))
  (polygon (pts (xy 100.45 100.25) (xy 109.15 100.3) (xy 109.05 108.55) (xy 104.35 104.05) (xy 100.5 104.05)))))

